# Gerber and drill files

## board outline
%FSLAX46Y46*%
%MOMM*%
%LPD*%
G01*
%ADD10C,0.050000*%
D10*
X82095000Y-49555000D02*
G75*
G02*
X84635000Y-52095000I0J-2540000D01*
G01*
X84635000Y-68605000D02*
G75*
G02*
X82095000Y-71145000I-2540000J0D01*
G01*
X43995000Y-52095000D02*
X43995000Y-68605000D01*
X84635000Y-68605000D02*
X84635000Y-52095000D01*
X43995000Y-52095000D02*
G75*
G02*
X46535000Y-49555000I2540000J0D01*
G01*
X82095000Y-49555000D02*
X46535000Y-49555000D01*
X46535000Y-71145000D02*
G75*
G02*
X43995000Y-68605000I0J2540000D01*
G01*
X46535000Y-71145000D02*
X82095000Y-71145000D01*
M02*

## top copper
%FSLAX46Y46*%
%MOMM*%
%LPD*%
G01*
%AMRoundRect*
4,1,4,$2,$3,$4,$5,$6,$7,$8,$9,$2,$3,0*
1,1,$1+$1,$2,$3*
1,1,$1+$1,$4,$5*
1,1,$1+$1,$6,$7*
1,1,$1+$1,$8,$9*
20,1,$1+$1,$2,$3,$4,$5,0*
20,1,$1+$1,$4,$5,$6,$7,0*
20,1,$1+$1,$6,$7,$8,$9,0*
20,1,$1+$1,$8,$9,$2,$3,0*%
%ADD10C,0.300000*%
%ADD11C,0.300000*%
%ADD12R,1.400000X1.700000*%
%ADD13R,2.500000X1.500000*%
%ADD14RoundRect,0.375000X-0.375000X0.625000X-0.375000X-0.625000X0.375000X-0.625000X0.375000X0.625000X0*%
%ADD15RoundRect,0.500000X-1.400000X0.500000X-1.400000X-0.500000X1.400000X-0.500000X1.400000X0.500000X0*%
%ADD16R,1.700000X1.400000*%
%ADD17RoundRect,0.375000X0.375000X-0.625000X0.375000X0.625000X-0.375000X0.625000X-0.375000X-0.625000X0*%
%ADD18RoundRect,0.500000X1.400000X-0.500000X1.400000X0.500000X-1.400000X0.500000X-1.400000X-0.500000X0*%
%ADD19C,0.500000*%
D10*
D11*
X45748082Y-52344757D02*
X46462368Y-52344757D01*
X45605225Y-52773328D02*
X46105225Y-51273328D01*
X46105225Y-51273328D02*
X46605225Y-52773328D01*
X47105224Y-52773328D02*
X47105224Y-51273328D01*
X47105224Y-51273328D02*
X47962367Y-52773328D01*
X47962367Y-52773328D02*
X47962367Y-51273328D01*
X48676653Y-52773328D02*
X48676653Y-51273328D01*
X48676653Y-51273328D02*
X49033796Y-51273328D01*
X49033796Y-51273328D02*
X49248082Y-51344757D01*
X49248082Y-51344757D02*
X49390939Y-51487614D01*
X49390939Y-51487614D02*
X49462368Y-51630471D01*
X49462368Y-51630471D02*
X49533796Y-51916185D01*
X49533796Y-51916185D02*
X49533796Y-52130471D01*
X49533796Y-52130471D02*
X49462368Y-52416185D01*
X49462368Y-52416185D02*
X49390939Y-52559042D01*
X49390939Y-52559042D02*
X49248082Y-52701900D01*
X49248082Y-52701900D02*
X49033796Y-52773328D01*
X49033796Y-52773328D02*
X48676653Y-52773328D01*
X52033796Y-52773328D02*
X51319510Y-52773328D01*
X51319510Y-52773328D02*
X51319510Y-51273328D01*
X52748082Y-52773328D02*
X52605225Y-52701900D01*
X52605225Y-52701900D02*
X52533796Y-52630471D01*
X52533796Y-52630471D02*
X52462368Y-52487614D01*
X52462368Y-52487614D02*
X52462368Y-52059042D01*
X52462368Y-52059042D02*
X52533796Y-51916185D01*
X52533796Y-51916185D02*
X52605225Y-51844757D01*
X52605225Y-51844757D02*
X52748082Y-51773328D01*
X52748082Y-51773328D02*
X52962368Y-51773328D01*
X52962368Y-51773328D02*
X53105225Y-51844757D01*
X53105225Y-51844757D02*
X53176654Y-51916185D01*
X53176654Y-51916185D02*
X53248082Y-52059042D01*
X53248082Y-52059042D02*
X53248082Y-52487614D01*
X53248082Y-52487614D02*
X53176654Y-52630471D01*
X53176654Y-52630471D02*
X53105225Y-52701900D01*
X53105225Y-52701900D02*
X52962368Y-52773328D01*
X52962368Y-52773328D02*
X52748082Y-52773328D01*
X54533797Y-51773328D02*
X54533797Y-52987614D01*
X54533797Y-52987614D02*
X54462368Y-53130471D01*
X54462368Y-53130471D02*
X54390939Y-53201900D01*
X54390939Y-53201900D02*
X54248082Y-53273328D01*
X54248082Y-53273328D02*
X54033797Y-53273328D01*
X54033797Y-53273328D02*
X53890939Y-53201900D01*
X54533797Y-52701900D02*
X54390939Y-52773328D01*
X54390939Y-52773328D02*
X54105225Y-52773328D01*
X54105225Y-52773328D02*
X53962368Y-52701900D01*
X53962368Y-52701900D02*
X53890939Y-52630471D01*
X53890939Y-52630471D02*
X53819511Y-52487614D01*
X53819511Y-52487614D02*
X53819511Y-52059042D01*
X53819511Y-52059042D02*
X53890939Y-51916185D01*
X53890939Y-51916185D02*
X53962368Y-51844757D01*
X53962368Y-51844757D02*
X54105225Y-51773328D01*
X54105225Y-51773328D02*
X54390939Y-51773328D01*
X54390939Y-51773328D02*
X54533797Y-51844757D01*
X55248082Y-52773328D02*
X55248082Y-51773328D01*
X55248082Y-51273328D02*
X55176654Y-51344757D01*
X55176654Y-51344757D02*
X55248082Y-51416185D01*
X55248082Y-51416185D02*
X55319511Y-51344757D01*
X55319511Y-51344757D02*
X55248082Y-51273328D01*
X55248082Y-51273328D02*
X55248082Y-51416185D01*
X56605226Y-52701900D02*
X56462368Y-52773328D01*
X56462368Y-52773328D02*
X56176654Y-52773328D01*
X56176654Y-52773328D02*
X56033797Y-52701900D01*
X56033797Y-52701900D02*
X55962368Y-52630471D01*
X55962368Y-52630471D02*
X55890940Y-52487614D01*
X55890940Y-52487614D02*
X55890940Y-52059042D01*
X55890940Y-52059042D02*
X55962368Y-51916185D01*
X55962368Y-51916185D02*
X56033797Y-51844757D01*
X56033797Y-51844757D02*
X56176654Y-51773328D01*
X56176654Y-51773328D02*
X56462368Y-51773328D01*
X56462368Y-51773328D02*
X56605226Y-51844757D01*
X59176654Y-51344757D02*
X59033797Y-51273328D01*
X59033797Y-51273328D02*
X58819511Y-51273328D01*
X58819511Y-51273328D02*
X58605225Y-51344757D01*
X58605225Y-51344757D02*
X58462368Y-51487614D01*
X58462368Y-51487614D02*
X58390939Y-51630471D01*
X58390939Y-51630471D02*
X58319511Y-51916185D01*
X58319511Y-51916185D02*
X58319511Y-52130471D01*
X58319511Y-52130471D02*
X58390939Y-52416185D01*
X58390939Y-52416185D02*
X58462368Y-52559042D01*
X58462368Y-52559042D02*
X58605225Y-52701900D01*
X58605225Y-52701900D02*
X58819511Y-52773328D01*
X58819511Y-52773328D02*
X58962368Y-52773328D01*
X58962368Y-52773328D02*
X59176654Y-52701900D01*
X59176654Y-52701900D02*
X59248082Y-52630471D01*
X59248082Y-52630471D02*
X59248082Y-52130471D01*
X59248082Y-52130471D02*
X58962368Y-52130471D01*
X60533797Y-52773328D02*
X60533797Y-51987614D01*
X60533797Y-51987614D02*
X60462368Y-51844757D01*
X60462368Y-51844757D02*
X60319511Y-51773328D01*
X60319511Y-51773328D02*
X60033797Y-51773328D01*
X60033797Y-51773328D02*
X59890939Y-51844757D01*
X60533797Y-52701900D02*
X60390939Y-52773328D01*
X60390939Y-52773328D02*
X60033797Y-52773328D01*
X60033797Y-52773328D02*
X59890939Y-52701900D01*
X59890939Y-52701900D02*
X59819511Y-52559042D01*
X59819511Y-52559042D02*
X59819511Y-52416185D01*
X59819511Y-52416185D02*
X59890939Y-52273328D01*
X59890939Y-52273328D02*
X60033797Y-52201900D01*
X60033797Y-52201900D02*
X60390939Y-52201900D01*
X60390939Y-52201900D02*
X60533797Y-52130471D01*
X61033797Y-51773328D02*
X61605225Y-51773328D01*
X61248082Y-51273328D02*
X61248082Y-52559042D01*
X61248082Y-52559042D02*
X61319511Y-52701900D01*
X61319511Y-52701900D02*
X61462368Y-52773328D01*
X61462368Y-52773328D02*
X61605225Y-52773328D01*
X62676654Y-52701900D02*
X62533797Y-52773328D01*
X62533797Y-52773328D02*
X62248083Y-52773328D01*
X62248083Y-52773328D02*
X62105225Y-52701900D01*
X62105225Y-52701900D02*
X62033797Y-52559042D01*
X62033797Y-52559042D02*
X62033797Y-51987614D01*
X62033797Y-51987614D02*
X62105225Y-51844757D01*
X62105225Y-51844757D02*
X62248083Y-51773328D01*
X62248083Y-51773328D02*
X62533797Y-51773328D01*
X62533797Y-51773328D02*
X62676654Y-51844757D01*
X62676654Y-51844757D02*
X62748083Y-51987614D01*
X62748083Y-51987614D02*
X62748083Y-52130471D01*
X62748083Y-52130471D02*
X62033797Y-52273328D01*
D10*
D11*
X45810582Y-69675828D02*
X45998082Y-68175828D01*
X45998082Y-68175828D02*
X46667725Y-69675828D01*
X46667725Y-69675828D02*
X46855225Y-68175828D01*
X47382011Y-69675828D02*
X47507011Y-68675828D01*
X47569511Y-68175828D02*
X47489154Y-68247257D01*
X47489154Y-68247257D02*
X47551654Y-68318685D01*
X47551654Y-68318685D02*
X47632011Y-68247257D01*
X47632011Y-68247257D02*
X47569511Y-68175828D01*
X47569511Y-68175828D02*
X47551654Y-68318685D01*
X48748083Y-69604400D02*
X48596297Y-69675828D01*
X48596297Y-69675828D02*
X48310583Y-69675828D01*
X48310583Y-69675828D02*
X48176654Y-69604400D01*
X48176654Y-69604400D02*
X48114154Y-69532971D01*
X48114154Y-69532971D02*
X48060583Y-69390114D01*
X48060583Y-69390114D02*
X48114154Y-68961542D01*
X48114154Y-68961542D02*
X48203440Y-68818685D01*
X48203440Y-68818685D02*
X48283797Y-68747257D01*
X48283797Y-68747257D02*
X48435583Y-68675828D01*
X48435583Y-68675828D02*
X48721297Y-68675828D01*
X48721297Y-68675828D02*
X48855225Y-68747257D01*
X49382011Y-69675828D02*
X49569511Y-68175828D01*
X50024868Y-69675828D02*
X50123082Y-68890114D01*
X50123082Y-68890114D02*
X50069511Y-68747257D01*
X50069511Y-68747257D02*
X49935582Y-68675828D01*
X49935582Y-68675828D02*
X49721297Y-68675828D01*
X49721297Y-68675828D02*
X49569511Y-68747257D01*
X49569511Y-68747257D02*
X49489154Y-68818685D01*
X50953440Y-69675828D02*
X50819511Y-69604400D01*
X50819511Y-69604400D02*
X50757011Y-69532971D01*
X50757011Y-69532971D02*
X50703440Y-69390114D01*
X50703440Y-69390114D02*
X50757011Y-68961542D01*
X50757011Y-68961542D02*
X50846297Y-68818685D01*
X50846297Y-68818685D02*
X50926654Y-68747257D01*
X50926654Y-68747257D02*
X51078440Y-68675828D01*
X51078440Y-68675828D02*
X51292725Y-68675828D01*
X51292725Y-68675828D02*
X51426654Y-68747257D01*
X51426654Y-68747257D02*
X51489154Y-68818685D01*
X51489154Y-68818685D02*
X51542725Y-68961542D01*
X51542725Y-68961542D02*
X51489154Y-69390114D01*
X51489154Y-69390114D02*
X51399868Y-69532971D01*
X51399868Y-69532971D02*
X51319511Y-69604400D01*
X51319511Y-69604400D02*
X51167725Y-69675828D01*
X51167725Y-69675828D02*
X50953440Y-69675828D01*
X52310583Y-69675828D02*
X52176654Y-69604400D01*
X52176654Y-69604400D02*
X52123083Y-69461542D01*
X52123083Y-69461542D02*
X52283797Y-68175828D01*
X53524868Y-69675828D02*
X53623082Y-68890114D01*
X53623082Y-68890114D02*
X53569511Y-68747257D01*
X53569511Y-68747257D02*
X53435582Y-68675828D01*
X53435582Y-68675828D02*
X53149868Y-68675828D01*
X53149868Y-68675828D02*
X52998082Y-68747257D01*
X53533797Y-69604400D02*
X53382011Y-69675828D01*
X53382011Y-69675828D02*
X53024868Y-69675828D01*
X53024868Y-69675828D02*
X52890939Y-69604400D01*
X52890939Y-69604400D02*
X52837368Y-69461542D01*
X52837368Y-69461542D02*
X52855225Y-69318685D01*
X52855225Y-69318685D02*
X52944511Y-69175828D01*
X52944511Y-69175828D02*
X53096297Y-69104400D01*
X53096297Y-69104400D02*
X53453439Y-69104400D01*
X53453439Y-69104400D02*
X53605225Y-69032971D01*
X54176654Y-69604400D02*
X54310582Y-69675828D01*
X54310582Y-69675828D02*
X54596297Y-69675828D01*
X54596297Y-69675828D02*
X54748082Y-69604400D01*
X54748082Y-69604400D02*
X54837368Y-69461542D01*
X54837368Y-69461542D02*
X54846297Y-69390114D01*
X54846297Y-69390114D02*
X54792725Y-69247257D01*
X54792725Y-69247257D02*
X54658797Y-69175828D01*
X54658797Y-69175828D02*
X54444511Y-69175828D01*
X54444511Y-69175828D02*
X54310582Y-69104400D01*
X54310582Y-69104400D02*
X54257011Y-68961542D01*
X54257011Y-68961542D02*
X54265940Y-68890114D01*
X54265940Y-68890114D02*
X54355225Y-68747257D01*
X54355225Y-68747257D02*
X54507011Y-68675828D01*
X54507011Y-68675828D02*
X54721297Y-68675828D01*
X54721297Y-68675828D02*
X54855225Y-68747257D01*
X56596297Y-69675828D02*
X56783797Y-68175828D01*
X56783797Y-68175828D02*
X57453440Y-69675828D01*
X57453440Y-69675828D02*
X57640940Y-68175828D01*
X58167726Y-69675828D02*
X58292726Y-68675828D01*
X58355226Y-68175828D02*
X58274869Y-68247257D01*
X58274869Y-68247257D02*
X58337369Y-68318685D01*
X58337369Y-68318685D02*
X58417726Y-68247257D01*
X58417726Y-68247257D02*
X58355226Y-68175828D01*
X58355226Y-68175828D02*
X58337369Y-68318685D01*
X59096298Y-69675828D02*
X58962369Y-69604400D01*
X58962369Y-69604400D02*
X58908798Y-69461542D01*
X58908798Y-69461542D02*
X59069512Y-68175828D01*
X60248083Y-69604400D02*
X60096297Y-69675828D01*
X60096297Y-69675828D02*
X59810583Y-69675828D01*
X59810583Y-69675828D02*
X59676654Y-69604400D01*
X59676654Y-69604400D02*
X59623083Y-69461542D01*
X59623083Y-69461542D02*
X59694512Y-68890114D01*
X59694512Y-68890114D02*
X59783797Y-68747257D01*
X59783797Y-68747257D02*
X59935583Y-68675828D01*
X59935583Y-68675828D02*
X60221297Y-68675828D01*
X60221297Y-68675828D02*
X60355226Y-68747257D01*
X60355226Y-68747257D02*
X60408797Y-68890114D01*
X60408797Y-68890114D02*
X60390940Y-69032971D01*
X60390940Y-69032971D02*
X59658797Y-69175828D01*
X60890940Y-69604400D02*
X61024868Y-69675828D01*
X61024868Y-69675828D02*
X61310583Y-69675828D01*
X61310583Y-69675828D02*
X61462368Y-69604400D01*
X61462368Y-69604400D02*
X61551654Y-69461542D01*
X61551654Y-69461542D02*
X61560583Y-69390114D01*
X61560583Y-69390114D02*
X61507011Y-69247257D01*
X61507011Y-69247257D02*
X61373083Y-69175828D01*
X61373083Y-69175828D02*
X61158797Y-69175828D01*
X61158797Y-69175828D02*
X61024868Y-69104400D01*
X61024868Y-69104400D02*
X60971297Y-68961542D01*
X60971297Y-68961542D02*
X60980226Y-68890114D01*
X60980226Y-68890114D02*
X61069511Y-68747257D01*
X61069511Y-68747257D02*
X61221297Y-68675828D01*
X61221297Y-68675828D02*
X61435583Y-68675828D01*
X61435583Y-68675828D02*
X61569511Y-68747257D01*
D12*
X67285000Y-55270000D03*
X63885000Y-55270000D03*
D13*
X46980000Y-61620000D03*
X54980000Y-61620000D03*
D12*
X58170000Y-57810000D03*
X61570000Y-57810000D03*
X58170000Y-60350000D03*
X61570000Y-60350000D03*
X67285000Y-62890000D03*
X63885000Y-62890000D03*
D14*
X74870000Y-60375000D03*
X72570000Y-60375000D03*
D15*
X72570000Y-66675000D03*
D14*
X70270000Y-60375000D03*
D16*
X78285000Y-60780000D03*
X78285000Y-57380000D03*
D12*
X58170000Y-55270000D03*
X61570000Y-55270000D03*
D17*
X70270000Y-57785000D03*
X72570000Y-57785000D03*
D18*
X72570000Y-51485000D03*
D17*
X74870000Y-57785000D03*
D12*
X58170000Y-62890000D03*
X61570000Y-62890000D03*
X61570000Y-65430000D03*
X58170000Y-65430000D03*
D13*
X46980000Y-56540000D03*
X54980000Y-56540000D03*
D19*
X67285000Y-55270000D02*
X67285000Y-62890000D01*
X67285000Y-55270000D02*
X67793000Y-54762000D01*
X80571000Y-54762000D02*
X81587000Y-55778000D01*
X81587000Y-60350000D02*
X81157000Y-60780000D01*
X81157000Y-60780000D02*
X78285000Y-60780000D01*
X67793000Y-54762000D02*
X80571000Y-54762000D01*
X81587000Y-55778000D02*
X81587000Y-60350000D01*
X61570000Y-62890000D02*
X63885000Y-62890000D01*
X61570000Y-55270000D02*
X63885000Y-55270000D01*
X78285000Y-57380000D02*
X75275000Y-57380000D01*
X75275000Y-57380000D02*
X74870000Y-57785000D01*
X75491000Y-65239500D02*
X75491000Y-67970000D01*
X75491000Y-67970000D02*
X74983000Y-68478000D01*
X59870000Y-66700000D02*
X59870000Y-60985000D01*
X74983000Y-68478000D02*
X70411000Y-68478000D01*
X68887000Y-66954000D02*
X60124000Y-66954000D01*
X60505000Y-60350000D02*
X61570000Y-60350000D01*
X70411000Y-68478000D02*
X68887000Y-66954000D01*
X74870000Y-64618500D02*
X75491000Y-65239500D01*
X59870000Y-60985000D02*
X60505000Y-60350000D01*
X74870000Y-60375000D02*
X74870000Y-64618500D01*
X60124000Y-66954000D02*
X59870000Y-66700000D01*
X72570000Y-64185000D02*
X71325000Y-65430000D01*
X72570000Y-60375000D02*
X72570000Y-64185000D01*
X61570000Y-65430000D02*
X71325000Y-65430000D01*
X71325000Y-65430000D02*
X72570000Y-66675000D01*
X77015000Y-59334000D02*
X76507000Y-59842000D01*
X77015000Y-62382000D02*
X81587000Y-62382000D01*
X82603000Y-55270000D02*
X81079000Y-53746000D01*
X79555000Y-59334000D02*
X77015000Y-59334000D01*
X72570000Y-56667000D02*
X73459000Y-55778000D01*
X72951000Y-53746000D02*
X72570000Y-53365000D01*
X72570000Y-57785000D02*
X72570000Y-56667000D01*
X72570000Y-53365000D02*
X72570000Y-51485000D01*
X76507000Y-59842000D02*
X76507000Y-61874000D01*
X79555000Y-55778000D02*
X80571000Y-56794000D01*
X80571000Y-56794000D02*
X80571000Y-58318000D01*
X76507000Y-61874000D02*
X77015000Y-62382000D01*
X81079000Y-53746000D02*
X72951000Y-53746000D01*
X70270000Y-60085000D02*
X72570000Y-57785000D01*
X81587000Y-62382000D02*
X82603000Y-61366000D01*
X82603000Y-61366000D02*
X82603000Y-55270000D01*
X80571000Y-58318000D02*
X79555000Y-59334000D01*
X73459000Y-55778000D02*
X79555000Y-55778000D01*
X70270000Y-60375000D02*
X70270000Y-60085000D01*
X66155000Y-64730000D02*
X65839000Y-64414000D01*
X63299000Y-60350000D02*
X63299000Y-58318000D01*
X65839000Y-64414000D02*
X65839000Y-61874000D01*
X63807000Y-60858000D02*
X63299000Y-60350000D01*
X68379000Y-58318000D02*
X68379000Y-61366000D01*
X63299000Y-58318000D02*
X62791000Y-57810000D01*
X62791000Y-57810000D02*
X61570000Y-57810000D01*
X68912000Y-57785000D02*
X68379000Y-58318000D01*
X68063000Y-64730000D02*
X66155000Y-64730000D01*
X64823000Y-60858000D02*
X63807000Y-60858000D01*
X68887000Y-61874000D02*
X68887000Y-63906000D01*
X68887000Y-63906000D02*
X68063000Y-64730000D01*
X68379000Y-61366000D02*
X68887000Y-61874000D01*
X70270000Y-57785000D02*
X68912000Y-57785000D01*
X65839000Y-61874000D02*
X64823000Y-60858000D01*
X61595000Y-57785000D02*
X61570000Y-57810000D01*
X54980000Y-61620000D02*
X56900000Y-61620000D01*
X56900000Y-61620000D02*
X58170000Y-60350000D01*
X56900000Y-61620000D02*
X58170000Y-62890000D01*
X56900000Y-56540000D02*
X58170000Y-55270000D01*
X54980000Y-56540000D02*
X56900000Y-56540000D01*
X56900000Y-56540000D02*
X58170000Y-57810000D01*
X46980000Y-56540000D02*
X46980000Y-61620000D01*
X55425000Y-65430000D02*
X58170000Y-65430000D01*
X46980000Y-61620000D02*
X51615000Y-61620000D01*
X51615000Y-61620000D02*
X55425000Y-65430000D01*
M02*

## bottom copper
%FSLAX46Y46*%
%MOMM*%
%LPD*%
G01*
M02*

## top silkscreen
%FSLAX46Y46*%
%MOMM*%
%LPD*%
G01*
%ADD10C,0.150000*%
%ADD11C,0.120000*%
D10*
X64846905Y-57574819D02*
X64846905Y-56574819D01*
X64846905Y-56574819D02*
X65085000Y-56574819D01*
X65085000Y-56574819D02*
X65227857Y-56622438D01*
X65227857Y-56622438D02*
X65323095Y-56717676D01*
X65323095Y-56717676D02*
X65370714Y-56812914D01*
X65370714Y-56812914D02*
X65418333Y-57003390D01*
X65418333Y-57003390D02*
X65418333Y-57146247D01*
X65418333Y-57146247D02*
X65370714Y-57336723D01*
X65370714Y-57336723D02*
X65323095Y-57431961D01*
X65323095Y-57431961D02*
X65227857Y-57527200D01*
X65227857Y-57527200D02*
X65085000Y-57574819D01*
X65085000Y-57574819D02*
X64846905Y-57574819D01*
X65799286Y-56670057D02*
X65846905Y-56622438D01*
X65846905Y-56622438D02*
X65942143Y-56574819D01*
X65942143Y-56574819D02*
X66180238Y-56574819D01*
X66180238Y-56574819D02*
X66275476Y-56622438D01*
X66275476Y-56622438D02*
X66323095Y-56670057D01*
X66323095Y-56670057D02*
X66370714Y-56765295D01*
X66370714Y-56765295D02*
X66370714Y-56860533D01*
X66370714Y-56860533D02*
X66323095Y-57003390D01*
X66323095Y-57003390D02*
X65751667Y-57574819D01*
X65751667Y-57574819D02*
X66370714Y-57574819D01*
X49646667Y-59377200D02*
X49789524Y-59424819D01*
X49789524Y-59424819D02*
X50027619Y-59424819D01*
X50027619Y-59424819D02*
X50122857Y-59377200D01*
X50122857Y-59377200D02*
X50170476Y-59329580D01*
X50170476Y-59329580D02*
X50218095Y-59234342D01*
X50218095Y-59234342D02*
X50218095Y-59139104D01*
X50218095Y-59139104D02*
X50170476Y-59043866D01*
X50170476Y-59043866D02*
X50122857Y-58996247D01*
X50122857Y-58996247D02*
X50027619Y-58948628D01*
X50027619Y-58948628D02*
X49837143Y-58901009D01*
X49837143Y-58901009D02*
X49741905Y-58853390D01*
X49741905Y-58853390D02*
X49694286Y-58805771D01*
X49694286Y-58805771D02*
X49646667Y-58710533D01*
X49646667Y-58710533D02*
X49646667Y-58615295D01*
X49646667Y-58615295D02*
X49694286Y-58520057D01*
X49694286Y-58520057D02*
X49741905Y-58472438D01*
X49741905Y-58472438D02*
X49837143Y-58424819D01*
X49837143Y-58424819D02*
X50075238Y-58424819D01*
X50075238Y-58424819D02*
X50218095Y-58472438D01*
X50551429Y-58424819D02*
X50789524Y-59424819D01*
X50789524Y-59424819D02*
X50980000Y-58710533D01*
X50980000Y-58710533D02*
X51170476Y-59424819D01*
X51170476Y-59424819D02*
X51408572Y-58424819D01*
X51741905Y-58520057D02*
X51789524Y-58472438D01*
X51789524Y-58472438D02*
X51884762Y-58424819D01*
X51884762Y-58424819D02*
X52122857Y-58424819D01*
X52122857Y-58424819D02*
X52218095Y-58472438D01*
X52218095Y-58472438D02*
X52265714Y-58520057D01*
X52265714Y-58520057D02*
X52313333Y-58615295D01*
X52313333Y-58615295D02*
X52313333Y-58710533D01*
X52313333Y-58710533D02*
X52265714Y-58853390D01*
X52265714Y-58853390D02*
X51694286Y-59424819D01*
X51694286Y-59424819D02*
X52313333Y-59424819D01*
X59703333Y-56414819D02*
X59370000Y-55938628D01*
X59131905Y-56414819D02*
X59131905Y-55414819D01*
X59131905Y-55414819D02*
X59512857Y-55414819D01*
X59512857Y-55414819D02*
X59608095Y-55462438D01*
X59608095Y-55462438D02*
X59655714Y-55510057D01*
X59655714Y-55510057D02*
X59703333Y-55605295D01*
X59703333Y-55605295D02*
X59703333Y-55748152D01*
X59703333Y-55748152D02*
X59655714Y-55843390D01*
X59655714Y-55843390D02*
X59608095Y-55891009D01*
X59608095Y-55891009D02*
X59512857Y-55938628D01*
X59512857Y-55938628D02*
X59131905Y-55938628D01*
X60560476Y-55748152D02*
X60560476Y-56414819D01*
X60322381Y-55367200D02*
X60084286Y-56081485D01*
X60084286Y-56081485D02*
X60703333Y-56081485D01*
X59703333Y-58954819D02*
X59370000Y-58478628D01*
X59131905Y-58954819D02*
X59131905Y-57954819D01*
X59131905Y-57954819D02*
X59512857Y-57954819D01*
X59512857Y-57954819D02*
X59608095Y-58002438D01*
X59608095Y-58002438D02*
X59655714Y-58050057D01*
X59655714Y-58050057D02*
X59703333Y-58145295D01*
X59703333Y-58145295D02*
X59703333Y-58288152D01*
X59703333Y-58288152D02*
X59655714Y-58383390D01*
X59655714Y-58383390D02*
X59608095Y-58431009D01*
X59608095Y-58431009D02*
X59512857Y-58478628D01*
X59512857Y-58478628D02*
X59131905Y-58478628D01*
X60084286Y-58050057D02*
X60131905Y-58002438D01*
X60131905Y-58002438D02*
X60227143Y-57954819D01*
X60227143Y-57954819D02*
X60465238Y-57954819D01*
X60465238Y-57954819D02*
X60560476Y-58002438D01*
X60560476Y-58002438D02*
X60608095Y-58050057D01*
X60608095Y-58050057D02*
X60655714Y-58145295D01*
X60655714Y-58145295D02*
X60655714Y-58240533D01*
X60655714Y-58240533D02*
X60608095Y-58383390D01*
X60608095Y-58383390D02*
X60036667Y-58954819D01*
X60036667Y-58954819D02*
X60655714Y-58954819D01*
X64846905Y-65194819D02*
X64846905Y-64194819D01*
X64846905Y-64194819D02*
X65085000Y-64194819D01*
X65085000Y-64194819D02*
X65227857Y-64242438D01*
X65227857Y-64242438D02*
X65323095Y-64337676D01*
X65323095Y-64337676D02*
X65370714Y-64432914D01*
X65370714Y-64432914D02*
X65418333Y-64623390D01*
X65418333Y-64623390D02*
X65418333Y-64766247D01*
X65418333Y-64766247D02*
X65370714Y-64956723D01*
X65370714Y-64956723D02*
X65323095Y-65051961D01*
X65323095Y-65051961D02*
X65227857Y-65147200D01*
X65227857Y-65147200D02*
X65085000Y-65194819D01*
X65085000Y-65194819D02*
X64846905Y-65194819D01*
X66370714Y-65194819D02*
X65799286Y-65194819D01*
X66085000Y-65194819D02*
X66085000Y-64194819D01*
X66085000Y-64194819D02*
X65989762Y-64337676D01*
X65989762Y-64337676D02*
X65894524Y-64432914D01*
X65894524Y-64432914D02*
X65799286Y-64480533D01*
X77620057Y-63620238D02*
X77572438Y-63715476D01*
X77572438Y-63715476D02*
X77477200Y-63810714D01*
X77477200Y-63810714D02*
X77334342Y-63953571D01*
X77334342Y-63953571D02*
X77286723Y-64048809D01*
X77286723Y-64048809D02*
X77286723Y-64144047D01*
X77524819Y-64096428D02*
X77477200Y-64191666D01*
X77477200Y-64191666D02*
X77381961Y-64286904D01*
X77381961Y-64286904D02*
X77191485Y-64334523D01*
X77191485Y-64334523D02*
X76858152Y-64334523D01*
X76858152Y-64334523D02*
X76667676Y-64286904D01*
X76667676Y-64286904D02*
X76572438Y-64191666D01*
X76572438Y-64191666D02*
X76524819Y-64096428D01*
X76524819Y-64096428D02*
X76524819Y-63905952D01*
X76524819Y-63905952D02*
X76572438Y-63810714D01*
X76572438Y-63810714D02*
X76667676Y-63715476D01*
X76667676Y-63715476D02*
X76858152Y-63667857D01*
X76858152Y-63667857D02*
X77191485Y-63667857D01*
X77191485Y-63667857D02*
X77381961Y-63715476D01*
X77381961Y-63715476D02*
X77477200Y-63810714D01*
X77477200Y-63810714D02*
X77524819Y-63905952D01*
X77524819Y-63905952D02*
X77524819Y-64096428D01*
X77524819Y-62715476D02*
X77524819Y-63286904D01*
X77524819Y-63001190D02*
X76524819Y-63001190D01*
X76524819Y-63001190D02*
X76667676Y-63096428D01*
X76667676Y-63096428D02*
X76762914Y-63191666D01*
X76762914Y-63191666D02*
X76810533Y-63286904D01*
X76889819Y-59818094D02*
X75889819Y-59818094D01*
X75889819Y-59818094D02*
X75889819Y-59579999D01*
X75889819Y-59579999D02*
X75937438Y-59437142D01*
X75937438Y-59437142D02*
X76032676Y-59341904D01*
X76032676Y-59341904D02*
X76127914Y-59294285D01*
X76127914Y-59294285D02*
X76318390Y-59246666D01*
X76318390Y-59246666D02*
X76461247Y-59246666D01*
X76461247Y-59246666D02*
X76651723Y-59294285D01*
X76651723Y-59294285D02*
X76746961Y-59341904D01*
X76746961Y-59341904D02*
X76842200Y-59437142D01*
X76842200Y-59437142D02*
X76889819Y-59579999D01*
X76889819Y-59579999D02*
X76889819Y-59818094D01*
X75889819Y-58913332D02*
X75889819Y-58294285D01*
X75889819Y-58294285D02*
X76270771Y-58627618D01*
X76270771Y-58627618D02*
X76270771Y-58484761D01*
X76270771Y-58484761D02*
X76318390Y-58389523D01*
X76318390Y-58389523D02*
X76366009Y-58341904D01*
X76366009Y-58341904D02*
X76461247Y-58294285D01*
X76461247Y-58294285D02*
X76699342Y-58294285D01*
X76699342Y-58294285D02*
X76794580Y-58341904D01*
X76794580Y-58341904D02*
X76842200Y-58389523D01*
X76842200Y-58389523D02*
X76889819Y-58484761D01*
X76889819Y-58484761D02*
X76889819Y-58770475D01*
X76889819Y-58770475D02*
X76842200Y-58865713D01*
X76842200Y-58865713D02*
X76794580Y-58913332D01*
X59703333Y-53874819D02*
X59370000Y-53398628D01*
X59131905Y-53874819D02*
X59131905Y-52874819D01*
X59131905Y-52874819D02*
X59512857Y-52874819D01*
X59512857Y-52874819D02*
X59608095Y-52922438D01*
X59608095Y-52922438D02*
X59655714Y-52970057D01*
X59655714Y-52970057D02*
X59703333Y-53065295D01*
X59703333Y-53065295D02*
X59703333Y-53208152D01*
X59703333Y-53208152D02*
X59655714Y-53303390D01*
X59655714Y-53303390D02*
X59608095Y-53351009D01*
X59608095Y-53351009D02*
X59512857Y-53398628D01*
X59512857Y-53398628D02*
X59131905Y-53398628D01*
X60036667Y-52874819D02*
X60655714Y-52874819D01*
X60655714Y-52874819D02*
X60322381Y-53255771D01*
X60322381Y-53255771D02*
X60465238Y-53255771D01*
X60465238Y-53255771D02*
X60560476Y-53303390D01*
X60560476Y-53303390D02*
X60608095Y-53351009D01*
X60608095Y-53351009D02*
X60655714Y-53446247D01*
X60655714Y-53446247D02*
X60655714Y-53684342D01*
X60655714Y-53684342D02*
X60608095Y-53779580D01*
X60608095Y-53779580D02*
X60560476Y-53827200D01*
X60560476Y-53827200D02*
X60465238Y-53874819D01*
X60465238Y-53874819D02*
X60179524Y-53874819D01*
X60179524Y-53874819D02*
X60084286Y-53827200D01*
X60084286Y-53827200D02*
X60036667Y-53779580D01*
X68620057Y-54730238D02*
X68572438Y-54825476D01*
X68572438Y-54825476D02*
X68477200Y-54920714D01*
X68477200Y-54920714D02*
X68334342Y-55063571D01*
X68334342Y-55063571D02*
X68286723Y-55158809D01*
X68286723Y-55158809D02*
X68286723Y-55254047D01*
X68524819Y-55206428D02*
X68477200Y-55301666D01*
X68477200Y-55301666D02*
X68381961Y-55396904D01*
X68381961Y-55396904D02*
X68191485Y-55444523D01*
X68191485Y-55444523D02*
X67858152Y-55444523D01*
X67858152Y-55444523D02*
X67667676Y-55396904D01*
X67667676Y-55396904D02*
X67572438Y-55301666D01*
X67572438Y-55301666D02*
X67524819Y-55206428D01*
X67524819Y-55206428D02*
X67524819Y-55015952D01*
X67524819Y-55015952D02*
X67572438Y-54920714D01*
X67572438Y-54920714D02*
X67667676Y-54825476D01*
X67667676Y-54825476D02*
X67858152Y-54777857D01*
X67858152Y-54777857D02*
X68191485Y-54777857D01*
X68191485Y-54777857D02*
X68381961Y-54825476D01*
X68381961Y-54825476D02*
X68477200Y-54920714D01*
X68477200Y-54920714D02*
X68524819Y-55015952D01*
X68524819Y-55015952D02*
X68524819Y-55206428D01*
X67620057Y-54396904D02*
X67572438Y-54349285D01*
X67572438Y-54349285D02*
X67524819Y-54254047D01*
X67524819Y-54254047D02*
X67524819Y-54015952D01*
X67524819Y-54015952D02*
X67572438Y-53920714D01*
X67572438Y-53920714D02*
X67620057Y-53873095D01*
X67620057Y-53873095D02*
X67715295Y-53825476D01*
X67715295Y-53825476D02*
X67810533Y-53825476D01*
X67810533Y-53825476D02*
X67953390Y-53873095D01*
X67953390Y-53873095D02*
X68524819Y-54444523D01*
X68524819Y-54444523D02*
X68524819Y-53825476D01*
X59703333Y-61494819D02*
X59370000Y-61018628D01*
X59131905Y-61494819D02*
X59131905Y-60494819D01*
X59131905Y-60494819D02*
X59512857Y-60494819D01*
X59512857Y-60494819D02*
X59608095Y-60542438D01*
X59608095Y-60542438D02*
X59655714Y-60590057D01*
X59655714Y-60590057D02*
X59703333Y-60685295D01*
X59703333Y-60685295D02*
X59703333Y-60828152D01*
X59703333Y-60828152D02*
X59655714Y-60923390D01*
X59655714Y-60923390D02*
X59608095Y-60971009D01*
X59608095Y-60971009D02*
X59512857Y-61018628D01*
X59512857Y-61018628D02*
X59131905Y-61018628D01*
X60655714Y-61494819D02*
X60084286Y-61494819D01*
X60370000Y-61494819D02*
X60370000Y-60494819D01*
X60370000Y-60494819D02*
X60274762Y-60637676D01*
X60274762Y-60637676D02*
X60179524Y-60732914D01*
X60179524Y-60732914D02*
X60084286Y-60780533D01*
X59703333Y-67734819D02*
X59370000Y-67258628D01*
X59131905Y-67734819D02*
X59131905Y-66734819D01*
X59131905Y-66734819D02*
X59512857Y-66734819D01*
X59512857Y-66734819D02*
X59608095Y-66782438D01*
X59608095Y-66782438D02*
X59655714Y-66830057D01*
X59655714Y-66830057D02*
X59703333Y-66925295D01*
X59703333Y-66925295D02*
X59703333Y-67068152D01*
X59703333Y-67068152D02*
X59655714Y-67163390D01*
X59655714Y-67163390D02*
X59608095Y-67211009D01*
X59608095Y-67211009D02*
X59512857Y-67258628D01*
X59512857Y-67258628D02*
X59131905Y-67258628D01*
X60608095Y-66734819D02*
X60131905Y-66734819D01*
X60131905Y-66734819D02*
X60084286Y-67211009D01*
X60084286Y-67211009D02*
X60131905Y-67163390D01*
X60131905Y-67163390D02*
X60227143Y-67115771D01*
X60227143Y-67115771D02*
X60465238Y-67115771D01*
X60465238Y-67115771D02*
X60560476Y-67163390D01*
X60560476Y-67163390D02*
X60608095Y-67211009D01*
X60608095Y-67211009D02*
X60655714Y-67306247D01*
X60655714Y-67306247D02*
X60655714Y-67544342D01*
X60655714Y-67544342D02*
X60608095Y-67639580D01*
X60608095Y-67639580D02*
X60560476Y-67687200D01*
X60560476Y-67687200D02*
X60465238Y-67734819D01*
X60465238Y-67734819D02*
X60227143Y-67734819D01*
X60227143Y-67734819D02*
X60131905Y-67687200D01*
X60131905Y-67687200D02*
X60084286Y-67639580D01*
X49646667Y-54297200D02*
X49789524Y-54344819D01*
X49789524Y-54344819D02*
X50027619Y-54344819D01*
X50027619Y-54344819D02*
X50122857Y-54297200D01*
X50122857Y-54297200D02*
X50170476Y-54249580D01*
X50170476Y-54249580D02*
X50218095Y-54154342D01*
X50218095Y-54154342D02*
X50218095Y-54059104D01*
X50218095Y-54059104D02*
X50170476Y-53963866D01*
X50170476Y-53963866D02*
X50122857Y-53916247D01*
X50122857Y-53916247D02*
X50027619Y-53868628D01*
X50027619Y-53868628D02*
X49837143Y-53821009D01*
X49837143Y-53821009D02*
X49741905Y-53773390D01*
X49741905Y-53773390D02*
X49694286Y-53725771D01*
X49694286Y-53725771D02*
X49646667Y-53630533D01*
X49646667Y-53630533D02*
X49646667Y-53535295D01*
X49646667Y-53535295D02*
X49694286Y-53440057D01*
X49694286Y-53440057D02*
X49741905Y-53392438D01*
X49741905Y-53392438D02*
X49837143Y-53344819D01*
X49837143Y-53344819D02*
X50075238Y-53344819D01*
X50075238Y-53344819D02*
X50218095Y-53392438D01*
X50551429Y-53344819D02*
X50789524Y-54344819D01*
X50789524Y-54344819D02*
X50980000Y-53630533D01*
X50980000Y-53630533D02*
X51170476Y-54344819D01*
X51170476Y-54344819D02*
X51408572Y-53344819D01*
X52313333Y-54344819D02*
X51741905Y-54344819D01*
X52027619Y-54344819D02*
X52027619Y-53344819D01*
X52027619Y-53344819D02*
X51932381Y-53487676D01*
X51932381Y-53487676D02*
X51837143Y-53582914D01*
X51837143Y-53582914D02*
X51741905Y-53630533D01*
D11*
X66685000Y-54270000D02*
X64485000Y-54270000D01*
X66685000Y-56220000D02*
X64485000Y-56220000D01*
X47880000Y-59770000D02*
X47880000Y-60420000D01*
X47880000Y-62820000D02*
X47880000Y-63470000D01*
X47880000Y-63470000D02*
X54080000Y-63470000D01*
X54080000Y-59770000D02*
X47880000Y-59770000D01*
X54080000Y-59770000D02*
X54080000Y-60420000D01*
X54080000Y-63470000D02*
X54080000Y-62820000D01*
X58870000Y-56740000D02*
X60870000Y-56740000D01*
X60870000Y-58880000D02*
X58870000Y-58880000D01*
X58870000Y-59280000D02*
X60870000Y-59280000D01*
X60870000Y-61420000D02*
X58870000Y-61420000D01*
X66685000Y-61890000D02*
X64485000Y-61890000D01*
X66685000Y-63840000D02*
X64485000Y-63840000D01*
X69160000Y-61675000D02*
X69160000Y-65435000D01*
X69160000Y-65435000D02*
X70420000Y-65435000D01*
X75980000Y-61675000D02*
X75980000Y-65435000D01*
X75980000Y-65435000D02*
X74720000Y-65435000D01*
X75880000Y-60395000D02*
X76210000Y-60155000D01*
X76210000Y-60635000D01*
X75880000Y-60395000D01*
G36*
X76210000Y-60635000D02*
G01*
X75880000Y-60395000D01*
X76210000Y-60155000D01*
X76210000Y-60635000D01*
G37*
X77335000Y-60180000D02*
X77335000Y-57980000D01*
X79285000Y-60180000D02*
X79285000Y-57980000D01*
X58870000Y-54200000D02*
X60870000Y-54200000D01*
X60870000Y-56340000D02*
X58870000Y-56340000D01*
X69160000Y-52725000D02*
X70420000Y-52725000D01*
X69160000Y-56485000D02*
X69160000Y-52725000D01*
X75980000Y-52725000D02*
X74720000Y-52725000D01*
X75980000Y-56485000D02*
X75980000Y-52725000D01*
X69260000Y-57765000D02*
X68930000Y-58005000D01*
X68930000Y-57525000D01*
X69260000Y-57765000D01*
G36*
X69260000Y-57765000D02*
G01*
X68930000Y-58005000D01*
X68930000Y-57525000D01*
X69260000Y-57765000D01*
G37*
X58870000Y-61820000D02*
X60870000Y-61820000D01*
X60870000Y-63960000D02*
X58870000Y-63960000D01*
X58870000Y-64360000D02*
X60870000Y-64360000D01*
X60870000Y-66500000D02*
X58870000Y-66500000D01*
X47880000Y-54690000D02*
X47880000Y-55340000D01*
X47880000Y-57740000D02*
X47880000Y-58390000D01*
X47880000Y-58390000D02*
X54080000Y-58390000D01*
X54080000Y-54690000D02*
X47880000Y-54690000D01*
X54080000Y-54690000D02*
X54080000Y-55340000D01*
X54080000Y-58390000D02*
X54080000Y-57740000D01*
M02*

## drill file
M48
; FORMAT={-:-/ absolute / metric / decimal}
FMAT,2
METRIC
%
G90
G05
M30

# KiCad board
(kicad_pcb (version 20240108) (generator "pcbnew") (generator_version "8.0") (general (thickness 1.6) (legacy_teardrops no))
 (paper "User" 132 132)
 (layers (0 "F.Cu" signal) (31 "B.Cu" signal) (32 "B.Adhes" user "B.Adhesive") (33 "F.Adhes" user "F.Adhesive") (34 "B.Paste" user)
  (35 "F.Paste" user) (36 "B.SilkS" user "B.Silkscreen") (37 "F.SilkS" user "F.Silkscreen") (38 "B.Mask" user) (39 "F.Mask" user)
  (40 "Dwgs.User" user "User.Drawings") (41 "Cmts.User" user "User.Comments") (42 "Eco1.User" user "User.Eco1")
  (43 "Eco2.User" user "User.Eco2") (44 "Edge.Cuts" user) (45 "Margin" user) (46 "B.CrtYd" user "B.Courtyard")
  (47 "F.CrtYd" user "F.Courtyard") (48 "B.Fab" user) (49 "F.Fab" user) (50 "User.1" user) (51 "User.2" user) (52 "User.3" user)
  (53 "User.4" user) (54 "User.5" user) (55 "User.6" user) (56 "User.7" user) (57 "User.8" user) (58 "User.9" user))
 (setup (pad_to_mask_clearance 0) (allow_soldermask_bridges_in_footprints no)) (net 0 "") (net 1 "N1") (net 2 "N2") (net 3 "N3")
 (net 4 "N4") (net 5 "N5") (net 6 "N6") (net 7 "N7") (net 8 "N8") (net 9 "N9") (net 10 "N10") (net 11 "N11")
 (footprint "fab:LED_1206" (layer "F.Cu") (at 65.585 55.27 180)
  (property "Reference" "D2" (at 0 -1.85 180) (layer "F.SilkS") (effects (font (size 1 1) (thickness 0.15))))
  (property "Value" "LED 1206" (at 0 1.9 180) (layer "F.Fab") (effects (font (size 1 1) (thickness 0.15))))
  (fp_line (start -1.1 1) (end 1.1 1) (stroke (width 0.12) (type solid)) (layer "F.SilkS"))
  (fp_line (start -1.1 -0.95) (end 1.1 -0.95) (stroke (width 0.12) (type solid)) (layer "F.SilkS"))
  (pad "1" smd rect (at -1.7 0 180) (size 1.4 1.7) (layers "F.Cu" "F.Paste" "F.Mask") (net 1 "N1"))
  (pad "2" smd rect (at 1.7 0 180) (size 1.4 1.7) (layers "F.Cu" "F.Paste" "F.Mask") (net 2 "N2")))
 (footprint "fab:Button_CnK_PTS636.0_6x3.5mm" (layer "F.Cu") (at 50.98 61.62)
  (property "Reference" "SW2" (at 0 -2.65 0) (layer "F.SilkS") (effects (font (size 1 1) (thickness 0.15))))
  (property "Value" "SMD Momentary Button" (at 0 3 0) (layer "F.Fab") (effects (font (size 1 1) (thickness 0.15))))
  (fp_line (start -3.1 -1.85) (end -3.1 -1.2) (stroke (width 0.12) (type solid)) (layer "F.SilkS"))
  (fp_line (start -3.1 1.2) (end -3.1 1.85) (stroke (width 0.12) (type solid)) (layer "F.SilkS"))
  (fp_line (start -3.1 1.85) (end 3.1 1.85) (stroke (width 0.12) (type solid)) (layer "F.SilkS"))
  (fp_line (start 3.1 -1.85) (end -3.1 -1.85) (stroke (width 0.12) (type solid)) (layer "F.SilkS"))
  (fp_line (start 3.1 -1.85) (end 3.1 -1.2) (stroke (width 0.12) (type solid)) (layer "F.SilkS"))
  (fp_line (start 3.1 1.85) (end 3.1 1.2) (stroke (width 0.12) (type solid)) (layer "F.SilkS"))
  (pad "1" smd rect (at -4 0) (size 2.5 1.5) (layers "F.Cu" "F.Paste" "F.Mask") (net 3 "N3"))
  (pad "2" smd rect (at 4 0) (size 2.5 1.5) (layers "F.Cu" "F.Paste" "F.Mask") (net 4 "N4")))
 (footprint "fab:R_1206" (layer "F.Cu") (at 59.87 57.81)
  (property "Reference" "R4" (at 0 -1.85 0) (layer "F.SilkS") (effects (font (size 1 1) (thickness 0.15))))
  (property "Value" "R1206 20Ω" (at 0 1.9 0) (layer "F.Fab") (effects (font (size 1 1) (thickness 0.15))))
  (fp_line (start -1 -1.07) (end 1 -1.07) (stroke (width 0.12) (type solid)) (layer "F.SilkS"))
  (fp_line (start 1 1.07) (end -1 1.07) (stroke (width 0.12) (type solid)) (layer "F.SilkS"))
  (pad "1" smd rect (at -1.7 0) (size 1.4 1.7) (layers "F.Cu" "F.Paste" "F.Mask") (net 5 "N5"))
  (pad "2" smd rect (at 1.7 0) (size 1.4 1.7) (layers "F.Cu" "F.Paste" "F.Mask") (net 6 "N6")))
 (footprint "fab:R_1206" (layer "F.Cu") (at 59.87 60.35)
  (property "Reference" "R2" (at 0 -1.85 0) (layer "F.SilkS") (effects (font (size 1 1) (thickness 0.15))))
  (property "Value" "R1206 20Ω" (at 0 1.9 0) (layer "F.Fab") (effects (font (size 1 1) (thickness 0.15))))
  (fp_line (start -1 -1.07) (end 1 -1.07) (stroke (width 0.12) (type solid)) (layer "F.SilkS"))
  (fp_line (start 1 1.07) (end -1 1.07) (stroke (width 0.12) (type solid)) (layer "F.SilkS"))
  (pad "1" smd rect (at -1.7 0) (size 1.4 1.7) (layers "F.Cu" "F.Paste" "F.Mask") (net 4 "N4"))
  (pad "2" smd rect (at 1.7 0) (size 1.4 1.7) (layers "F.Cu" "F.Paste" "F.Mask") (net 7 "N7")))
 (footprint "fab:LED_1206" (layer "F.Cu") (at 65.585 62.89 180)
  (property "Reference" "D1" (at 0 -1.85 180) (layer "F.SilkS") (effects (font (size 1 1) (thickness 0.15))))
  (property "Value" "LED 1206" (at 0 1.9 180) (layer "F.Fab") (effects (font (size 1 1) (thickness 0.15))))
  (fp_line (start -1.1 1) (end 1.1 1) (stroke (width 0.12) (type solid)) (layer "F.SilkS"))
  (fp_line (start -1.1 -0.95) (end 1.1 -0.95) (stroke (width 0.12) (type solid)) (layer "F.SilkS"))
  (pad "1" smd rect (at -1.7 0 180) (size 1.4 1.7) (layers "F.Cu" "F.Paste" "F.Mask") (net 1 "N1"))
  (pad "2" smd rect (at 1.7 0 180) (size 1.4 1.7) (layers "F.Cu" "F.Paste" "F.Mask") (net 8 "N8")))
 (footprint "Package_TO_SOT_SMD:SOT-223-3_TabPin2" (layer "F.Cu") (at 72.57 63.525 -90)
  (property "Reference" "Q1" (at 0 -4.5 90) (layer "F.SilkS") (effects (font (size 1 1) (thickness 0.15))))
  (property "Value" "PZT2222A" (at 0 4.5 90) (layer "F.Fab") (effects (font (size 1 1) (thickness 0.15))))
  (fp_line (start -1.85 3.41) (end 1.91 3.41) (stroke (width 0.12) (type solid)) (layer "F.SilkS"))
  (fp_line (start 1.91 3.41) (end 1.91 2.15) (stroke (width 0.12) (type solid)) (layer "F.SilkS"))
  (fp_line (start -1.85 -3.41) (end 1.91 -3.41) (stroke (width 0.12) (type solid)) (layer "F.SilkS"))
  (fp_line (start 1.91 -3.41) (end 1.91 -2.15) (stroke (width 0.12) (type solid)) (layer "F.SilkS"))
  (fp_poly
   (pts (xy -3.13 -3.31) (xy -3.37 -3.64) (xy -2.89 -3.64) (xy -3.13 -3.31)) (stroke (width 0.12) (type solid)) (fill solid)
   (layer "F.SilkS"))
  (pad "1" smd roundrect (at -3.15 -2.3 270) (size 2 1.5) (layers "F.Cu" "F.Paste" "F.Mask") (roundrect_rratio 0.25) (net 7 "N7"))
  (pad "2" smd roundrect (at -3.15 0 270) (size 2 1.5) (layers "F.Cu" "F.Paste" "F.Mask") (roundrect_rratio 0.25) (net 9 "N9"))
  (pad "2" smd roundrect (at 3.15 0 270) (size 2 3.8) (layers "F.Cu" "F.Paste" "F.Mask") (roundrect_rratio 0.25) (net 9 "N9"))
  (pad "3" smd roundrect (at -3.15 2.3 270) (size 2 1.5) (layers "F.Cu" "F.Paste" "F.Mask") (roundrect_rratio 0.25) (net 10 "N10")))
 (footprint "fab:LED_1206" (layer "F.Cu") (at 78.285 59.08 90)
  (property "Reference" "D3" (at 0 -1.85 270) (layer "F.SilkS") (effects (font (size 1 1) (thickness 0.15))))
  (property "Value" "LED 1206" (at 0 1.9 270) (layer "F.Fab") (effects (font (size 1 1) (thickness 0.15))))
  (fp_line (start -1.1 -0.95) (end 1.1 -0.95) (stroke (width 0.12) (type solid)) (layer "F.SilkS"))
  (fp_line (start -1.1 1) (end 1.1 1) (stroke (width 0.12) (type solid)) (layer "F.SilkS"))
  (pad "1" smd rect (at -1.7 0 90) (size 1.4 1.7) (layers "F.Cu" "F.Paste" "F.Mask") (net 1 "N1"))
  (pad "2" smd rect (at 1.7 0 90) (size 1.4 1.7) (layers "F.Cu" "F.Paste" "F.Mask") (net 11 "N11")))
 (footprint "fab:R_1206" (layer "F.Cu") (at 59.87 55.27)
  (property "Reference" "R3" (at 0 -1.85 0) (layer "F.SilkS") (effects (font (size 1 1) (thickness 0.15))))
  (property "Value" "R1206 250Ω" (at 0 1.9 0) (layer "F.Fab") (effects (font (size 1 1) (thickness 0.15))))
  (fp_line (start -1 -1.07) (end 1 -1.07) (stroke (width 0.12) (type solid)) (layer "F.SilkS"))
  (fp_line (start 1 1.07) (end -1 1.07) (stroke (width 0.12) (type solid)) (layer "F.SilkS"))
  (pad "1" smd rect (at -1.7 0) (size 1.4 1.7) (layers "F.Cu" "F.Paste" "F.Mask") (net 5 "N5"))
  (pad "2" smd rect (at 1.7 0) (size 1.4 1.7) (layers "F.Cu" "F.Paste" "F.Mask") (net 2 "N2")))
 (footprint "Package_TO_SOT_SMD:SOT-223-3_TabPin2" (layer "F.Cu") (at 72.57 54.635 90)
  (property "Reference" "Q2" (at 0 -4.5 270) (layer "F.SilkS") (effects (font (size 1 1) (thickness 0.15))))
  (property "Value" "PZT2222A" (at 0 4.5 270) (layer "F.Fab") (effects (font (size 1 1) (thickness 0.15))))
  (fp_line (start 1.91 -3.41) (end 1.91 -2.15) (stroke (width 0.12) (type solid)) (layer "F.SilkS"))
  (fp_line (start -1.85 -3.41) (end 1.91 -3.41) (stroke (width 0.12) (type solid)) (layer "F.SilkS"))
  (fp_line (start 1.91 3.41) (end 1.91 2.15) (stroke (width 0.12) (type solid)) (layer "F.SilkS"))
  (fp_line (start -1.85 3.41) (end 1.91 3.41) (stroke (width 0.12) (type solid)) (layer "F.SilkS"))
  (fp_poly
   (pts (xy -3.13 -3.31) (xy -3.37 -3.64) (xy -2.89 -3.64) (xy -3.13 -3.31)) (stroke (width 0.12) (type solid)) (fill solid)
   (layer "F.SilkS"))
  (pad "1" smd roundrect (at -3.15 -2.3 90) (size 2 1.5) (layers "F.Cu" "F.Paste" "F.Mask") (roundrect_rratio 0.25) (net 6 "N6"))
  (pad "2" smd roundrect (at -3.15 0 90) (size 2 1.5) (layers "F.Cu" "F.Paste" "F.Mask") (roundrect_rratio 0.25) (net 10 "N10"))
  (pad "2" smd roundrect (at 3.15 0 90) (size 2 3.8) (layers "F.Cu" "F.Paste" "F.Mask") (roundrect_rratio 0.25) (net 10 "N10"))
  (pad "3" smd roundrect (at -3.15 2.3 90) (size 2 1.5) (layers "F.Cu" "F.Paste" "F.Mask") (roundrect_rratio 0.25) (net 11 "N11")))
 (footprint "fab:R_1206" (layer "F.Cu") (at 59.87 62.89)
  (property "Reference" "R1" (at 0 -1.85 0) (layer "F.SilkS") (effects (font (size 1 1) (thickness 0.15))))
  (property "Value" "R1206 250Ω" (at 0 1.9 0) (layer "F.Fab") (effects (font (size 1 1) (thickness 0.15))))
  (fp_line (start -1 -1.07) (end 1 -1.07) (stroke (width 0.12) (type solid)) (layer "F.SilkS"))
  (fp_line (start 1 1.07) (end -1 1.07) (stroke (width 0.12) (type solid)) (layer "F.SilkS"))
  (pad "1" smd rect (at -1.7 0) (size 1.4 1.7) (layers "F.Cu" "F.Paste" "F.Mask") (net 4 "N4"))
  (pad "2" smd rect (at 1.7 0) (size 1.4 1.7) (layers "F.Cu" "F.Paste" "F.Mask") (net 8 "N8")))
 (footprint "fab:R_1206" (layer "F.Cu") (at 59.87 65.43 180)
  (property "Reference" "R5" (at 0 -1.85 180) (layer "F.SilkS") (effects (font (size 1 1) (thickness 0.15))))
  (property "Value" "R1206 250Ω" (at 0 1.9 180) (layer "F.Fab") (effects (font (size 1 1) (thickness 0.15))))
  (fp_line (start 1 1.07) (end -1 1.07) (stroke (width 0.12) (type solid)) (layer "F.SilkS"))
  (fp_line (start -1 -1.07) (end 1 -1.07) (stroke (width 0.12) (type solid)) (layer "F.SilkS"))
  (pad "1" smd rect (at -1.7 0 180) (size 1.4 1.7) (layers "F.Cu" "F.Paste" "F.Mask") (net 9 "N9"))
  (pad "2" smd rect (at 1.7 0 180) (size 1.4 1.7) (layers "F.Cu" "F.Paste" "F.Mask") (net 3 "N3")))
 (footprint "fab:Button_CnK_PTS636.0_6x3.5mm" (layer "F.Cu") (at 50.98 56.54)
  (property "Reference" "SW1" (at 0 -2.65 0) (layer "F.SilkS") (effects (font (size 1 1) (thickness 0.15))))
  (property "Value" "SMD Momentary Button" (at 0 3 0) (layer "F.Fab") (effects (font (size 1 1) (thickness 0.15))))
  (fp_line (start -3.1 -1.85) (end -3.1 -1.2) (stroke (width 0.12) (type solid)) (layer "F.SilkS"))
  (fp_line (start -3.1 1.2) (end -3.1 1.85) (stroke (width 0.12) (type solid)) (layer "F.SilkS"))
  (fp_line (start -3.1 1.85) (end 3.1 1.85) (stroke (width 0.12) (type solid)) (layer "F.SilkS"))
  (fp_line (start 3.1 -1.85) (end -3.1 -1.85) (stroke (width 0.12) (type solid)) (layer "F.SilkS"))
  (fp_line (start 3.1 -1.85) (end 3.1 -1.2) (stroke (width 0.12) (type solid)) (layer "F.SilkS"))
  (fp_line (start 3.1 1.85) (end 3.1 1.2) (stroke (width 0.12) (type solid)) (layer "F.SilkS"))
  (pad "1" smd rect (at -4 0) (size 2.5 1.5) (layers "F.Cu" "F.Paste" "F.Mask") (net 3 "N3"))
  (pad "2" smd rect (at 4 0) (size 2.5 1.5) (layers "F.Cu" "F.Paste" "F.Mask") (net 5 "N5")))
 (gr_arc (start 82.095 49.555) (mid 83.891051 50.298949) (end 84.635 52.095) (stroke (width 0.05) (type default)) (layer "Edge.Cuts"))
 (gr_arc (start 84.635 68.605) (mid 83.891051 70.401051) (end 82.095 71.145) (stroke (width 0.05) (type default)) (layer "Edge.Cuts"))
 (gr_line (start 43.995 52.095) (end 43.995 68.605) (stroke (width 0.05) (type default)) (layer "Edge.Cuts"))
 (gr_line (start 84.635 68.605) (end 84.635 52.095) (stroke (width 0.05) (type default)) (layer "Edge.Cuts"))
 (gr_arc (start 43.995 52.095) (mid 44.738949 50.298949) (end 46.535 49.555) (stroke (width 0.05) (type default)) (layer "Edge.Cuts"))
 (gr_line (start 82.095 49.555) (end 46.535 49.555) (stroke (width 0.05) (type default)) (layer "Edge.Cuts"))
 (gr_arc (start 46.535 71.145) (mid 44.738949 70.401051) (end 43.995 68.605) (stroke (width 0.05) (type default)) (layer "Edge.Cuts"))
 (gr_line (start 46.535 71.145) (end 82.095 71.145) (stroke (width 0.05) (type default)) (layer "Edge.Cuts"))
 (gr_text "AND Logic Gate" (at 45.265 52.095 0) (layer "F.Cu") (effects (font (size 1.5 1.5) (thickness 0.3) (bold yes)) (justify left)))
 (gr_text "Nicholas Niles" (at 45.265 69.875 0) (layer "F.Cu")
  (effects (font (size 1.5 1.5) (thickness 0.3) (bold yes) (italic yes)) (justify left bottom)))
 (segment (start 67.285 55.27) (end 67.285 62.89) (width 0.5) (layer "F.Cu") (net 1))
 (segment (start 67.285 55.27) (end 67.793 54.762) (width 0.5) (layer "F.Cu") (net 1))
 (segment (start 80.571 54.762) (end 81.587 55.778) (width 0.5) (layer "F.Cu") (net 1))
 (segment (start 81.587 60.35) (end 81.157 60.78) (width 0.5) (layer "F.Cu") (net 1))
 (segment (start 81.157 60.78) (end 78.285 60.78) (width 0.5) (layer "F.Cu") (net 1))
 (segment (start 67.793 54.762) (end 80.571 54.762) (width 0.5) (layer "F.Cu") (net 1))
 (segment (start 81.587 55.778) (end 81.587 60.35) (width 0.5) (layer "F.Cu") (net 1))
 (segment (start 61.57 62.89) (end 63.885 62.89) (width 0.5) (layer "F.Cu") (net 8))
 (segment (start 61.57 55.27) (end 63.885 55.27) (width 0.5) (layer "F.Cu") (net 2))
 (segment (start 78.285 57.38) (end 75.275 57.38) (width 0.5) (layer "F.Cu") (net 11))
 (segment (start 75.275 57.38) (end 74.87 57.785) (width 0.5) (layer "F.Cu") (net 11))
 (segment (start 75.491 65.2395) (end 75.491 67.97) (width 0.5) (layer "F.Cu") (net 7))
 (segment (start 75.491 67.97) (end 74.983 68.478) (width 0.5) (layer "F.Cu") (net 7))
 (segment (start 59.87 66.7) (end 59.87 60.985) (width 0.5) (layer "F.Cu") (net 7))
 (segment (start 74.983 68.478) (end 70.411 68.478) (width 0.5) (layer "F.Cu") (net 7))
 (segment (start 68.887 66.954) (end 60.124 66.954) (width 0.5) (layer "F.Cu") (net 7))
 (segment (start 60.505 60.35) (end 61.57 60.35) (width 0.5) (layer "F.Cu") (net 7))
 (segment (start 70.411 68.478) (end 68.887 66.954) (width 0.5) (layer "F.Cu") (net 7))
 (segment (start 74.87 64.6185) (end 75.491 65.2395) (width 0.5) (layer "F.Cu") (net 7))
 (segment (start 59.87 60.985) (end 60.505 60.35) (width 0.5) (layer "F.Cu") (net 7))
 (segment (start 74.87 60.375) (end 74.87 64.6185) (width 0.5) (layer "F.Cu") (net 7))
 (segment (start 60.124 66.954) (end 59.87 66.7) (width 0.5) (layer "F.Cu") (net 7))
 (segment (start 72.57 64.185) (end 71.325 65.43) (width 0.5) (layer "F.Cu") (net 9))
 (segment (start 72.57 60.375) (end 72.57 64.185) (width 0.5) (layer "F.Cu") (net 9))
 (segment (start 61.57 65.43) (end 71.325 65.43) (width 0.5) (layer "F.Cu") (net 9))
 (segment (start 71.325 65.43) (end 72.57 66.675) (width 0.5) (layer "F.Cu") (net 9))
 (segment (start 77.015 59.334) (end 76.507 59.842) (width 0.5) (layer "F.Cu") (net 10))
 (segment (start 77.015 62.382) (end 81.587 62.382) (width 0.5) (layer "F.Cu") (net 10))
 (segment (start 82.603 55.27) (end 81.079 53.746) (width 0.5) (layer "F.Cu") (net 10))
 (segment (start 79.555 59.334) (end 77.015 59.334) (width 0.5) (layer "F.Cu") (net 10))
 (segment (start 72.57 56.667) (end 73.459 55.778) (width 0.5) (layer "F.Cu") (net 10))
 (segment (start 72.951 53.746) (end 72.57 53.365) (width 0.5) (layer "F.Cu") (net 10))
 (segment (start 72.57 57.785) (end 72.57 56.667) (width 0.5) (layer "F.Cu") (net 10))
 (segment (start 72.57 53.365) (end 72.57 51.485) (width 0.5) (layer "F.Cu") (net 10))
 (segment (start 76.507 59.842) (end 76.507 61.874) (width 0.5) (layer "F.Cu") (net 10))
 (segment (start 79.555 55.778) (end 80.571 56.794) (width 0.5) (layer "F.Cu") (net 10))
 (segment (start 80.571 56.794) (end 80.571 58.318) (width 0.5) (layer "F.Cu") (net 10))
 (segment (start 76.507 61.874) (end 77.015 62.382) (width 0.5) (layer "F.Cu") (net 10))
 (segment (start 81.079 53.746) (end 72.951 53.746) (width 0.5) (layer "F.Cu") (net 10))
 (segment (start 70.27 60.085) (end 72.57 57.785) (width 0.5) (layer "F.Cu") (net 10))
 (segment (start 81.587 62.382) (end 82.603 61.366) (width 0.5) (layer "F.Cu") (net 10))
 (segment (start 82.603 61.366) (end 82.603 55.27) (width 0.5) (layer "F.Cu") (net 10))
 (segment (start 80.571 58.318) (end 79.555 59.334) (width 0.5) (layer "F.Cu") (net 10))
 (segment (start 73.459 55.778) (end 79.555 55.778) (width 0.5) (layer "F.Cu") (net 10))
 (segment (start 70.27 60.375) (end 70.27 60.085) (width 0.5) (layer "F.Cu") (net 10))
 (segment (start 66.155 64.73) (end 65.839 64.414) (width 0.5) (layer "F.Cu") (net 6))
 (segment (start 63.299 60.35) (end 63.299 58.318) (width 0.5) (layer "F.Cu") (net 6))
 (segment (start 65.839 64.414) (end 65.839 61.874) (width 0.5) (layer "F.Cu") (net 6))
 (segment (start 63.807 60.858) (end 63.299 60.35) (width 0.5) (layer "F.Cu") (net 6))
 (segment (start 68.379 58.318) (end 68.379 61.366) (width 0.5) (layer "F.Cu") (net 6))
 (segment (start 63.299 58.318) (end 62.791 57.81) (width 0.5) (layer "F.Cu") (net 6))
 (segment (start 62.791 57.81) (end 61.57 57.81) (width 0.5) (layer "F.Cu") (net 6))
 (segment (start 68.912 57.785) (end 68.379 58.318) (width 0.5) (layer "F.Cu") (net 6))
 (segment (start 68.063 64.73) (end 66.155 64.73) (width 0.5) (layer "F.Cu") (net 6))
 (segment (start 64.823 60.858) (end 63.807 60.858) (width 0.5) (layer "F.Cu") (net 6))
 (segment (start 68.887 61.874) (end 68.887 63.906) (width 0.5) (layer "F.Cu") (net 6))
 (segment (start 68.887 63.906) (end 68.063 64.73) (width 0.5) (layer "F.Cu") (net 6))
 (segment (start 68.379 61.366) (end 68.887 61.874) (width 0.5) (layer "F.Cu") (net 6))
 (segment (start 70.27 57.785) (end 68.912 57.785) (width 0.5) (layer "F.Cu") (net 6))
 (segment (start 65.839 61.874) (end 64.823 60.858) (width 0.5) (layer "F.Cu") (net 6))
 (segment (start 61.595 57.785) (end 61.57 57.81) (width 0.5) (layer "F.Cu") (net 6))
 (segment (start 54.98 61.62) (end 56.9 61.62) (width 0.5) (layer "F.Cu") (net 4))
 (segment (start 56.9 61.62) (end 58.17 60.35) (width 0.5) (layer "F.Cu") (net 4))
 (segment (start 56.9 61.62) (end 58.17 62.89) (width 0.5) (layer "F.Cu") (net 4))
 (segment (start 56.9 56.54) (end 58.17 55.27) (width 0.5) (layer "F.Cu") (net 5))
 (segment (start 54.98 56.54) (end 56.9 56.54) (width 0.5) (layer "F.Cu") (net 5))
 (segment (start 56.9 56.54) (end 58.17 57.81) (width 0.5) (layer "F.Cu") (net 5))
 (segment (start 46.98 56.54) (end 46.98 61.62) (width 0.5) (layer "F.Cu") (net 3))
 (segment (start 55.425 65.43) (end 58.17 65.43) (width 0.5) (layer "F.Cu") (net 3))
 (segment (start 46.98 61.62) (end 51.615 61.62) (width 0.5) (layer "F.Cu") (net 3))
 (segment (start 51.615 61.62) (end 55.425 65.43) (width 0.5) (layer "F.Cu") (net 3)))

